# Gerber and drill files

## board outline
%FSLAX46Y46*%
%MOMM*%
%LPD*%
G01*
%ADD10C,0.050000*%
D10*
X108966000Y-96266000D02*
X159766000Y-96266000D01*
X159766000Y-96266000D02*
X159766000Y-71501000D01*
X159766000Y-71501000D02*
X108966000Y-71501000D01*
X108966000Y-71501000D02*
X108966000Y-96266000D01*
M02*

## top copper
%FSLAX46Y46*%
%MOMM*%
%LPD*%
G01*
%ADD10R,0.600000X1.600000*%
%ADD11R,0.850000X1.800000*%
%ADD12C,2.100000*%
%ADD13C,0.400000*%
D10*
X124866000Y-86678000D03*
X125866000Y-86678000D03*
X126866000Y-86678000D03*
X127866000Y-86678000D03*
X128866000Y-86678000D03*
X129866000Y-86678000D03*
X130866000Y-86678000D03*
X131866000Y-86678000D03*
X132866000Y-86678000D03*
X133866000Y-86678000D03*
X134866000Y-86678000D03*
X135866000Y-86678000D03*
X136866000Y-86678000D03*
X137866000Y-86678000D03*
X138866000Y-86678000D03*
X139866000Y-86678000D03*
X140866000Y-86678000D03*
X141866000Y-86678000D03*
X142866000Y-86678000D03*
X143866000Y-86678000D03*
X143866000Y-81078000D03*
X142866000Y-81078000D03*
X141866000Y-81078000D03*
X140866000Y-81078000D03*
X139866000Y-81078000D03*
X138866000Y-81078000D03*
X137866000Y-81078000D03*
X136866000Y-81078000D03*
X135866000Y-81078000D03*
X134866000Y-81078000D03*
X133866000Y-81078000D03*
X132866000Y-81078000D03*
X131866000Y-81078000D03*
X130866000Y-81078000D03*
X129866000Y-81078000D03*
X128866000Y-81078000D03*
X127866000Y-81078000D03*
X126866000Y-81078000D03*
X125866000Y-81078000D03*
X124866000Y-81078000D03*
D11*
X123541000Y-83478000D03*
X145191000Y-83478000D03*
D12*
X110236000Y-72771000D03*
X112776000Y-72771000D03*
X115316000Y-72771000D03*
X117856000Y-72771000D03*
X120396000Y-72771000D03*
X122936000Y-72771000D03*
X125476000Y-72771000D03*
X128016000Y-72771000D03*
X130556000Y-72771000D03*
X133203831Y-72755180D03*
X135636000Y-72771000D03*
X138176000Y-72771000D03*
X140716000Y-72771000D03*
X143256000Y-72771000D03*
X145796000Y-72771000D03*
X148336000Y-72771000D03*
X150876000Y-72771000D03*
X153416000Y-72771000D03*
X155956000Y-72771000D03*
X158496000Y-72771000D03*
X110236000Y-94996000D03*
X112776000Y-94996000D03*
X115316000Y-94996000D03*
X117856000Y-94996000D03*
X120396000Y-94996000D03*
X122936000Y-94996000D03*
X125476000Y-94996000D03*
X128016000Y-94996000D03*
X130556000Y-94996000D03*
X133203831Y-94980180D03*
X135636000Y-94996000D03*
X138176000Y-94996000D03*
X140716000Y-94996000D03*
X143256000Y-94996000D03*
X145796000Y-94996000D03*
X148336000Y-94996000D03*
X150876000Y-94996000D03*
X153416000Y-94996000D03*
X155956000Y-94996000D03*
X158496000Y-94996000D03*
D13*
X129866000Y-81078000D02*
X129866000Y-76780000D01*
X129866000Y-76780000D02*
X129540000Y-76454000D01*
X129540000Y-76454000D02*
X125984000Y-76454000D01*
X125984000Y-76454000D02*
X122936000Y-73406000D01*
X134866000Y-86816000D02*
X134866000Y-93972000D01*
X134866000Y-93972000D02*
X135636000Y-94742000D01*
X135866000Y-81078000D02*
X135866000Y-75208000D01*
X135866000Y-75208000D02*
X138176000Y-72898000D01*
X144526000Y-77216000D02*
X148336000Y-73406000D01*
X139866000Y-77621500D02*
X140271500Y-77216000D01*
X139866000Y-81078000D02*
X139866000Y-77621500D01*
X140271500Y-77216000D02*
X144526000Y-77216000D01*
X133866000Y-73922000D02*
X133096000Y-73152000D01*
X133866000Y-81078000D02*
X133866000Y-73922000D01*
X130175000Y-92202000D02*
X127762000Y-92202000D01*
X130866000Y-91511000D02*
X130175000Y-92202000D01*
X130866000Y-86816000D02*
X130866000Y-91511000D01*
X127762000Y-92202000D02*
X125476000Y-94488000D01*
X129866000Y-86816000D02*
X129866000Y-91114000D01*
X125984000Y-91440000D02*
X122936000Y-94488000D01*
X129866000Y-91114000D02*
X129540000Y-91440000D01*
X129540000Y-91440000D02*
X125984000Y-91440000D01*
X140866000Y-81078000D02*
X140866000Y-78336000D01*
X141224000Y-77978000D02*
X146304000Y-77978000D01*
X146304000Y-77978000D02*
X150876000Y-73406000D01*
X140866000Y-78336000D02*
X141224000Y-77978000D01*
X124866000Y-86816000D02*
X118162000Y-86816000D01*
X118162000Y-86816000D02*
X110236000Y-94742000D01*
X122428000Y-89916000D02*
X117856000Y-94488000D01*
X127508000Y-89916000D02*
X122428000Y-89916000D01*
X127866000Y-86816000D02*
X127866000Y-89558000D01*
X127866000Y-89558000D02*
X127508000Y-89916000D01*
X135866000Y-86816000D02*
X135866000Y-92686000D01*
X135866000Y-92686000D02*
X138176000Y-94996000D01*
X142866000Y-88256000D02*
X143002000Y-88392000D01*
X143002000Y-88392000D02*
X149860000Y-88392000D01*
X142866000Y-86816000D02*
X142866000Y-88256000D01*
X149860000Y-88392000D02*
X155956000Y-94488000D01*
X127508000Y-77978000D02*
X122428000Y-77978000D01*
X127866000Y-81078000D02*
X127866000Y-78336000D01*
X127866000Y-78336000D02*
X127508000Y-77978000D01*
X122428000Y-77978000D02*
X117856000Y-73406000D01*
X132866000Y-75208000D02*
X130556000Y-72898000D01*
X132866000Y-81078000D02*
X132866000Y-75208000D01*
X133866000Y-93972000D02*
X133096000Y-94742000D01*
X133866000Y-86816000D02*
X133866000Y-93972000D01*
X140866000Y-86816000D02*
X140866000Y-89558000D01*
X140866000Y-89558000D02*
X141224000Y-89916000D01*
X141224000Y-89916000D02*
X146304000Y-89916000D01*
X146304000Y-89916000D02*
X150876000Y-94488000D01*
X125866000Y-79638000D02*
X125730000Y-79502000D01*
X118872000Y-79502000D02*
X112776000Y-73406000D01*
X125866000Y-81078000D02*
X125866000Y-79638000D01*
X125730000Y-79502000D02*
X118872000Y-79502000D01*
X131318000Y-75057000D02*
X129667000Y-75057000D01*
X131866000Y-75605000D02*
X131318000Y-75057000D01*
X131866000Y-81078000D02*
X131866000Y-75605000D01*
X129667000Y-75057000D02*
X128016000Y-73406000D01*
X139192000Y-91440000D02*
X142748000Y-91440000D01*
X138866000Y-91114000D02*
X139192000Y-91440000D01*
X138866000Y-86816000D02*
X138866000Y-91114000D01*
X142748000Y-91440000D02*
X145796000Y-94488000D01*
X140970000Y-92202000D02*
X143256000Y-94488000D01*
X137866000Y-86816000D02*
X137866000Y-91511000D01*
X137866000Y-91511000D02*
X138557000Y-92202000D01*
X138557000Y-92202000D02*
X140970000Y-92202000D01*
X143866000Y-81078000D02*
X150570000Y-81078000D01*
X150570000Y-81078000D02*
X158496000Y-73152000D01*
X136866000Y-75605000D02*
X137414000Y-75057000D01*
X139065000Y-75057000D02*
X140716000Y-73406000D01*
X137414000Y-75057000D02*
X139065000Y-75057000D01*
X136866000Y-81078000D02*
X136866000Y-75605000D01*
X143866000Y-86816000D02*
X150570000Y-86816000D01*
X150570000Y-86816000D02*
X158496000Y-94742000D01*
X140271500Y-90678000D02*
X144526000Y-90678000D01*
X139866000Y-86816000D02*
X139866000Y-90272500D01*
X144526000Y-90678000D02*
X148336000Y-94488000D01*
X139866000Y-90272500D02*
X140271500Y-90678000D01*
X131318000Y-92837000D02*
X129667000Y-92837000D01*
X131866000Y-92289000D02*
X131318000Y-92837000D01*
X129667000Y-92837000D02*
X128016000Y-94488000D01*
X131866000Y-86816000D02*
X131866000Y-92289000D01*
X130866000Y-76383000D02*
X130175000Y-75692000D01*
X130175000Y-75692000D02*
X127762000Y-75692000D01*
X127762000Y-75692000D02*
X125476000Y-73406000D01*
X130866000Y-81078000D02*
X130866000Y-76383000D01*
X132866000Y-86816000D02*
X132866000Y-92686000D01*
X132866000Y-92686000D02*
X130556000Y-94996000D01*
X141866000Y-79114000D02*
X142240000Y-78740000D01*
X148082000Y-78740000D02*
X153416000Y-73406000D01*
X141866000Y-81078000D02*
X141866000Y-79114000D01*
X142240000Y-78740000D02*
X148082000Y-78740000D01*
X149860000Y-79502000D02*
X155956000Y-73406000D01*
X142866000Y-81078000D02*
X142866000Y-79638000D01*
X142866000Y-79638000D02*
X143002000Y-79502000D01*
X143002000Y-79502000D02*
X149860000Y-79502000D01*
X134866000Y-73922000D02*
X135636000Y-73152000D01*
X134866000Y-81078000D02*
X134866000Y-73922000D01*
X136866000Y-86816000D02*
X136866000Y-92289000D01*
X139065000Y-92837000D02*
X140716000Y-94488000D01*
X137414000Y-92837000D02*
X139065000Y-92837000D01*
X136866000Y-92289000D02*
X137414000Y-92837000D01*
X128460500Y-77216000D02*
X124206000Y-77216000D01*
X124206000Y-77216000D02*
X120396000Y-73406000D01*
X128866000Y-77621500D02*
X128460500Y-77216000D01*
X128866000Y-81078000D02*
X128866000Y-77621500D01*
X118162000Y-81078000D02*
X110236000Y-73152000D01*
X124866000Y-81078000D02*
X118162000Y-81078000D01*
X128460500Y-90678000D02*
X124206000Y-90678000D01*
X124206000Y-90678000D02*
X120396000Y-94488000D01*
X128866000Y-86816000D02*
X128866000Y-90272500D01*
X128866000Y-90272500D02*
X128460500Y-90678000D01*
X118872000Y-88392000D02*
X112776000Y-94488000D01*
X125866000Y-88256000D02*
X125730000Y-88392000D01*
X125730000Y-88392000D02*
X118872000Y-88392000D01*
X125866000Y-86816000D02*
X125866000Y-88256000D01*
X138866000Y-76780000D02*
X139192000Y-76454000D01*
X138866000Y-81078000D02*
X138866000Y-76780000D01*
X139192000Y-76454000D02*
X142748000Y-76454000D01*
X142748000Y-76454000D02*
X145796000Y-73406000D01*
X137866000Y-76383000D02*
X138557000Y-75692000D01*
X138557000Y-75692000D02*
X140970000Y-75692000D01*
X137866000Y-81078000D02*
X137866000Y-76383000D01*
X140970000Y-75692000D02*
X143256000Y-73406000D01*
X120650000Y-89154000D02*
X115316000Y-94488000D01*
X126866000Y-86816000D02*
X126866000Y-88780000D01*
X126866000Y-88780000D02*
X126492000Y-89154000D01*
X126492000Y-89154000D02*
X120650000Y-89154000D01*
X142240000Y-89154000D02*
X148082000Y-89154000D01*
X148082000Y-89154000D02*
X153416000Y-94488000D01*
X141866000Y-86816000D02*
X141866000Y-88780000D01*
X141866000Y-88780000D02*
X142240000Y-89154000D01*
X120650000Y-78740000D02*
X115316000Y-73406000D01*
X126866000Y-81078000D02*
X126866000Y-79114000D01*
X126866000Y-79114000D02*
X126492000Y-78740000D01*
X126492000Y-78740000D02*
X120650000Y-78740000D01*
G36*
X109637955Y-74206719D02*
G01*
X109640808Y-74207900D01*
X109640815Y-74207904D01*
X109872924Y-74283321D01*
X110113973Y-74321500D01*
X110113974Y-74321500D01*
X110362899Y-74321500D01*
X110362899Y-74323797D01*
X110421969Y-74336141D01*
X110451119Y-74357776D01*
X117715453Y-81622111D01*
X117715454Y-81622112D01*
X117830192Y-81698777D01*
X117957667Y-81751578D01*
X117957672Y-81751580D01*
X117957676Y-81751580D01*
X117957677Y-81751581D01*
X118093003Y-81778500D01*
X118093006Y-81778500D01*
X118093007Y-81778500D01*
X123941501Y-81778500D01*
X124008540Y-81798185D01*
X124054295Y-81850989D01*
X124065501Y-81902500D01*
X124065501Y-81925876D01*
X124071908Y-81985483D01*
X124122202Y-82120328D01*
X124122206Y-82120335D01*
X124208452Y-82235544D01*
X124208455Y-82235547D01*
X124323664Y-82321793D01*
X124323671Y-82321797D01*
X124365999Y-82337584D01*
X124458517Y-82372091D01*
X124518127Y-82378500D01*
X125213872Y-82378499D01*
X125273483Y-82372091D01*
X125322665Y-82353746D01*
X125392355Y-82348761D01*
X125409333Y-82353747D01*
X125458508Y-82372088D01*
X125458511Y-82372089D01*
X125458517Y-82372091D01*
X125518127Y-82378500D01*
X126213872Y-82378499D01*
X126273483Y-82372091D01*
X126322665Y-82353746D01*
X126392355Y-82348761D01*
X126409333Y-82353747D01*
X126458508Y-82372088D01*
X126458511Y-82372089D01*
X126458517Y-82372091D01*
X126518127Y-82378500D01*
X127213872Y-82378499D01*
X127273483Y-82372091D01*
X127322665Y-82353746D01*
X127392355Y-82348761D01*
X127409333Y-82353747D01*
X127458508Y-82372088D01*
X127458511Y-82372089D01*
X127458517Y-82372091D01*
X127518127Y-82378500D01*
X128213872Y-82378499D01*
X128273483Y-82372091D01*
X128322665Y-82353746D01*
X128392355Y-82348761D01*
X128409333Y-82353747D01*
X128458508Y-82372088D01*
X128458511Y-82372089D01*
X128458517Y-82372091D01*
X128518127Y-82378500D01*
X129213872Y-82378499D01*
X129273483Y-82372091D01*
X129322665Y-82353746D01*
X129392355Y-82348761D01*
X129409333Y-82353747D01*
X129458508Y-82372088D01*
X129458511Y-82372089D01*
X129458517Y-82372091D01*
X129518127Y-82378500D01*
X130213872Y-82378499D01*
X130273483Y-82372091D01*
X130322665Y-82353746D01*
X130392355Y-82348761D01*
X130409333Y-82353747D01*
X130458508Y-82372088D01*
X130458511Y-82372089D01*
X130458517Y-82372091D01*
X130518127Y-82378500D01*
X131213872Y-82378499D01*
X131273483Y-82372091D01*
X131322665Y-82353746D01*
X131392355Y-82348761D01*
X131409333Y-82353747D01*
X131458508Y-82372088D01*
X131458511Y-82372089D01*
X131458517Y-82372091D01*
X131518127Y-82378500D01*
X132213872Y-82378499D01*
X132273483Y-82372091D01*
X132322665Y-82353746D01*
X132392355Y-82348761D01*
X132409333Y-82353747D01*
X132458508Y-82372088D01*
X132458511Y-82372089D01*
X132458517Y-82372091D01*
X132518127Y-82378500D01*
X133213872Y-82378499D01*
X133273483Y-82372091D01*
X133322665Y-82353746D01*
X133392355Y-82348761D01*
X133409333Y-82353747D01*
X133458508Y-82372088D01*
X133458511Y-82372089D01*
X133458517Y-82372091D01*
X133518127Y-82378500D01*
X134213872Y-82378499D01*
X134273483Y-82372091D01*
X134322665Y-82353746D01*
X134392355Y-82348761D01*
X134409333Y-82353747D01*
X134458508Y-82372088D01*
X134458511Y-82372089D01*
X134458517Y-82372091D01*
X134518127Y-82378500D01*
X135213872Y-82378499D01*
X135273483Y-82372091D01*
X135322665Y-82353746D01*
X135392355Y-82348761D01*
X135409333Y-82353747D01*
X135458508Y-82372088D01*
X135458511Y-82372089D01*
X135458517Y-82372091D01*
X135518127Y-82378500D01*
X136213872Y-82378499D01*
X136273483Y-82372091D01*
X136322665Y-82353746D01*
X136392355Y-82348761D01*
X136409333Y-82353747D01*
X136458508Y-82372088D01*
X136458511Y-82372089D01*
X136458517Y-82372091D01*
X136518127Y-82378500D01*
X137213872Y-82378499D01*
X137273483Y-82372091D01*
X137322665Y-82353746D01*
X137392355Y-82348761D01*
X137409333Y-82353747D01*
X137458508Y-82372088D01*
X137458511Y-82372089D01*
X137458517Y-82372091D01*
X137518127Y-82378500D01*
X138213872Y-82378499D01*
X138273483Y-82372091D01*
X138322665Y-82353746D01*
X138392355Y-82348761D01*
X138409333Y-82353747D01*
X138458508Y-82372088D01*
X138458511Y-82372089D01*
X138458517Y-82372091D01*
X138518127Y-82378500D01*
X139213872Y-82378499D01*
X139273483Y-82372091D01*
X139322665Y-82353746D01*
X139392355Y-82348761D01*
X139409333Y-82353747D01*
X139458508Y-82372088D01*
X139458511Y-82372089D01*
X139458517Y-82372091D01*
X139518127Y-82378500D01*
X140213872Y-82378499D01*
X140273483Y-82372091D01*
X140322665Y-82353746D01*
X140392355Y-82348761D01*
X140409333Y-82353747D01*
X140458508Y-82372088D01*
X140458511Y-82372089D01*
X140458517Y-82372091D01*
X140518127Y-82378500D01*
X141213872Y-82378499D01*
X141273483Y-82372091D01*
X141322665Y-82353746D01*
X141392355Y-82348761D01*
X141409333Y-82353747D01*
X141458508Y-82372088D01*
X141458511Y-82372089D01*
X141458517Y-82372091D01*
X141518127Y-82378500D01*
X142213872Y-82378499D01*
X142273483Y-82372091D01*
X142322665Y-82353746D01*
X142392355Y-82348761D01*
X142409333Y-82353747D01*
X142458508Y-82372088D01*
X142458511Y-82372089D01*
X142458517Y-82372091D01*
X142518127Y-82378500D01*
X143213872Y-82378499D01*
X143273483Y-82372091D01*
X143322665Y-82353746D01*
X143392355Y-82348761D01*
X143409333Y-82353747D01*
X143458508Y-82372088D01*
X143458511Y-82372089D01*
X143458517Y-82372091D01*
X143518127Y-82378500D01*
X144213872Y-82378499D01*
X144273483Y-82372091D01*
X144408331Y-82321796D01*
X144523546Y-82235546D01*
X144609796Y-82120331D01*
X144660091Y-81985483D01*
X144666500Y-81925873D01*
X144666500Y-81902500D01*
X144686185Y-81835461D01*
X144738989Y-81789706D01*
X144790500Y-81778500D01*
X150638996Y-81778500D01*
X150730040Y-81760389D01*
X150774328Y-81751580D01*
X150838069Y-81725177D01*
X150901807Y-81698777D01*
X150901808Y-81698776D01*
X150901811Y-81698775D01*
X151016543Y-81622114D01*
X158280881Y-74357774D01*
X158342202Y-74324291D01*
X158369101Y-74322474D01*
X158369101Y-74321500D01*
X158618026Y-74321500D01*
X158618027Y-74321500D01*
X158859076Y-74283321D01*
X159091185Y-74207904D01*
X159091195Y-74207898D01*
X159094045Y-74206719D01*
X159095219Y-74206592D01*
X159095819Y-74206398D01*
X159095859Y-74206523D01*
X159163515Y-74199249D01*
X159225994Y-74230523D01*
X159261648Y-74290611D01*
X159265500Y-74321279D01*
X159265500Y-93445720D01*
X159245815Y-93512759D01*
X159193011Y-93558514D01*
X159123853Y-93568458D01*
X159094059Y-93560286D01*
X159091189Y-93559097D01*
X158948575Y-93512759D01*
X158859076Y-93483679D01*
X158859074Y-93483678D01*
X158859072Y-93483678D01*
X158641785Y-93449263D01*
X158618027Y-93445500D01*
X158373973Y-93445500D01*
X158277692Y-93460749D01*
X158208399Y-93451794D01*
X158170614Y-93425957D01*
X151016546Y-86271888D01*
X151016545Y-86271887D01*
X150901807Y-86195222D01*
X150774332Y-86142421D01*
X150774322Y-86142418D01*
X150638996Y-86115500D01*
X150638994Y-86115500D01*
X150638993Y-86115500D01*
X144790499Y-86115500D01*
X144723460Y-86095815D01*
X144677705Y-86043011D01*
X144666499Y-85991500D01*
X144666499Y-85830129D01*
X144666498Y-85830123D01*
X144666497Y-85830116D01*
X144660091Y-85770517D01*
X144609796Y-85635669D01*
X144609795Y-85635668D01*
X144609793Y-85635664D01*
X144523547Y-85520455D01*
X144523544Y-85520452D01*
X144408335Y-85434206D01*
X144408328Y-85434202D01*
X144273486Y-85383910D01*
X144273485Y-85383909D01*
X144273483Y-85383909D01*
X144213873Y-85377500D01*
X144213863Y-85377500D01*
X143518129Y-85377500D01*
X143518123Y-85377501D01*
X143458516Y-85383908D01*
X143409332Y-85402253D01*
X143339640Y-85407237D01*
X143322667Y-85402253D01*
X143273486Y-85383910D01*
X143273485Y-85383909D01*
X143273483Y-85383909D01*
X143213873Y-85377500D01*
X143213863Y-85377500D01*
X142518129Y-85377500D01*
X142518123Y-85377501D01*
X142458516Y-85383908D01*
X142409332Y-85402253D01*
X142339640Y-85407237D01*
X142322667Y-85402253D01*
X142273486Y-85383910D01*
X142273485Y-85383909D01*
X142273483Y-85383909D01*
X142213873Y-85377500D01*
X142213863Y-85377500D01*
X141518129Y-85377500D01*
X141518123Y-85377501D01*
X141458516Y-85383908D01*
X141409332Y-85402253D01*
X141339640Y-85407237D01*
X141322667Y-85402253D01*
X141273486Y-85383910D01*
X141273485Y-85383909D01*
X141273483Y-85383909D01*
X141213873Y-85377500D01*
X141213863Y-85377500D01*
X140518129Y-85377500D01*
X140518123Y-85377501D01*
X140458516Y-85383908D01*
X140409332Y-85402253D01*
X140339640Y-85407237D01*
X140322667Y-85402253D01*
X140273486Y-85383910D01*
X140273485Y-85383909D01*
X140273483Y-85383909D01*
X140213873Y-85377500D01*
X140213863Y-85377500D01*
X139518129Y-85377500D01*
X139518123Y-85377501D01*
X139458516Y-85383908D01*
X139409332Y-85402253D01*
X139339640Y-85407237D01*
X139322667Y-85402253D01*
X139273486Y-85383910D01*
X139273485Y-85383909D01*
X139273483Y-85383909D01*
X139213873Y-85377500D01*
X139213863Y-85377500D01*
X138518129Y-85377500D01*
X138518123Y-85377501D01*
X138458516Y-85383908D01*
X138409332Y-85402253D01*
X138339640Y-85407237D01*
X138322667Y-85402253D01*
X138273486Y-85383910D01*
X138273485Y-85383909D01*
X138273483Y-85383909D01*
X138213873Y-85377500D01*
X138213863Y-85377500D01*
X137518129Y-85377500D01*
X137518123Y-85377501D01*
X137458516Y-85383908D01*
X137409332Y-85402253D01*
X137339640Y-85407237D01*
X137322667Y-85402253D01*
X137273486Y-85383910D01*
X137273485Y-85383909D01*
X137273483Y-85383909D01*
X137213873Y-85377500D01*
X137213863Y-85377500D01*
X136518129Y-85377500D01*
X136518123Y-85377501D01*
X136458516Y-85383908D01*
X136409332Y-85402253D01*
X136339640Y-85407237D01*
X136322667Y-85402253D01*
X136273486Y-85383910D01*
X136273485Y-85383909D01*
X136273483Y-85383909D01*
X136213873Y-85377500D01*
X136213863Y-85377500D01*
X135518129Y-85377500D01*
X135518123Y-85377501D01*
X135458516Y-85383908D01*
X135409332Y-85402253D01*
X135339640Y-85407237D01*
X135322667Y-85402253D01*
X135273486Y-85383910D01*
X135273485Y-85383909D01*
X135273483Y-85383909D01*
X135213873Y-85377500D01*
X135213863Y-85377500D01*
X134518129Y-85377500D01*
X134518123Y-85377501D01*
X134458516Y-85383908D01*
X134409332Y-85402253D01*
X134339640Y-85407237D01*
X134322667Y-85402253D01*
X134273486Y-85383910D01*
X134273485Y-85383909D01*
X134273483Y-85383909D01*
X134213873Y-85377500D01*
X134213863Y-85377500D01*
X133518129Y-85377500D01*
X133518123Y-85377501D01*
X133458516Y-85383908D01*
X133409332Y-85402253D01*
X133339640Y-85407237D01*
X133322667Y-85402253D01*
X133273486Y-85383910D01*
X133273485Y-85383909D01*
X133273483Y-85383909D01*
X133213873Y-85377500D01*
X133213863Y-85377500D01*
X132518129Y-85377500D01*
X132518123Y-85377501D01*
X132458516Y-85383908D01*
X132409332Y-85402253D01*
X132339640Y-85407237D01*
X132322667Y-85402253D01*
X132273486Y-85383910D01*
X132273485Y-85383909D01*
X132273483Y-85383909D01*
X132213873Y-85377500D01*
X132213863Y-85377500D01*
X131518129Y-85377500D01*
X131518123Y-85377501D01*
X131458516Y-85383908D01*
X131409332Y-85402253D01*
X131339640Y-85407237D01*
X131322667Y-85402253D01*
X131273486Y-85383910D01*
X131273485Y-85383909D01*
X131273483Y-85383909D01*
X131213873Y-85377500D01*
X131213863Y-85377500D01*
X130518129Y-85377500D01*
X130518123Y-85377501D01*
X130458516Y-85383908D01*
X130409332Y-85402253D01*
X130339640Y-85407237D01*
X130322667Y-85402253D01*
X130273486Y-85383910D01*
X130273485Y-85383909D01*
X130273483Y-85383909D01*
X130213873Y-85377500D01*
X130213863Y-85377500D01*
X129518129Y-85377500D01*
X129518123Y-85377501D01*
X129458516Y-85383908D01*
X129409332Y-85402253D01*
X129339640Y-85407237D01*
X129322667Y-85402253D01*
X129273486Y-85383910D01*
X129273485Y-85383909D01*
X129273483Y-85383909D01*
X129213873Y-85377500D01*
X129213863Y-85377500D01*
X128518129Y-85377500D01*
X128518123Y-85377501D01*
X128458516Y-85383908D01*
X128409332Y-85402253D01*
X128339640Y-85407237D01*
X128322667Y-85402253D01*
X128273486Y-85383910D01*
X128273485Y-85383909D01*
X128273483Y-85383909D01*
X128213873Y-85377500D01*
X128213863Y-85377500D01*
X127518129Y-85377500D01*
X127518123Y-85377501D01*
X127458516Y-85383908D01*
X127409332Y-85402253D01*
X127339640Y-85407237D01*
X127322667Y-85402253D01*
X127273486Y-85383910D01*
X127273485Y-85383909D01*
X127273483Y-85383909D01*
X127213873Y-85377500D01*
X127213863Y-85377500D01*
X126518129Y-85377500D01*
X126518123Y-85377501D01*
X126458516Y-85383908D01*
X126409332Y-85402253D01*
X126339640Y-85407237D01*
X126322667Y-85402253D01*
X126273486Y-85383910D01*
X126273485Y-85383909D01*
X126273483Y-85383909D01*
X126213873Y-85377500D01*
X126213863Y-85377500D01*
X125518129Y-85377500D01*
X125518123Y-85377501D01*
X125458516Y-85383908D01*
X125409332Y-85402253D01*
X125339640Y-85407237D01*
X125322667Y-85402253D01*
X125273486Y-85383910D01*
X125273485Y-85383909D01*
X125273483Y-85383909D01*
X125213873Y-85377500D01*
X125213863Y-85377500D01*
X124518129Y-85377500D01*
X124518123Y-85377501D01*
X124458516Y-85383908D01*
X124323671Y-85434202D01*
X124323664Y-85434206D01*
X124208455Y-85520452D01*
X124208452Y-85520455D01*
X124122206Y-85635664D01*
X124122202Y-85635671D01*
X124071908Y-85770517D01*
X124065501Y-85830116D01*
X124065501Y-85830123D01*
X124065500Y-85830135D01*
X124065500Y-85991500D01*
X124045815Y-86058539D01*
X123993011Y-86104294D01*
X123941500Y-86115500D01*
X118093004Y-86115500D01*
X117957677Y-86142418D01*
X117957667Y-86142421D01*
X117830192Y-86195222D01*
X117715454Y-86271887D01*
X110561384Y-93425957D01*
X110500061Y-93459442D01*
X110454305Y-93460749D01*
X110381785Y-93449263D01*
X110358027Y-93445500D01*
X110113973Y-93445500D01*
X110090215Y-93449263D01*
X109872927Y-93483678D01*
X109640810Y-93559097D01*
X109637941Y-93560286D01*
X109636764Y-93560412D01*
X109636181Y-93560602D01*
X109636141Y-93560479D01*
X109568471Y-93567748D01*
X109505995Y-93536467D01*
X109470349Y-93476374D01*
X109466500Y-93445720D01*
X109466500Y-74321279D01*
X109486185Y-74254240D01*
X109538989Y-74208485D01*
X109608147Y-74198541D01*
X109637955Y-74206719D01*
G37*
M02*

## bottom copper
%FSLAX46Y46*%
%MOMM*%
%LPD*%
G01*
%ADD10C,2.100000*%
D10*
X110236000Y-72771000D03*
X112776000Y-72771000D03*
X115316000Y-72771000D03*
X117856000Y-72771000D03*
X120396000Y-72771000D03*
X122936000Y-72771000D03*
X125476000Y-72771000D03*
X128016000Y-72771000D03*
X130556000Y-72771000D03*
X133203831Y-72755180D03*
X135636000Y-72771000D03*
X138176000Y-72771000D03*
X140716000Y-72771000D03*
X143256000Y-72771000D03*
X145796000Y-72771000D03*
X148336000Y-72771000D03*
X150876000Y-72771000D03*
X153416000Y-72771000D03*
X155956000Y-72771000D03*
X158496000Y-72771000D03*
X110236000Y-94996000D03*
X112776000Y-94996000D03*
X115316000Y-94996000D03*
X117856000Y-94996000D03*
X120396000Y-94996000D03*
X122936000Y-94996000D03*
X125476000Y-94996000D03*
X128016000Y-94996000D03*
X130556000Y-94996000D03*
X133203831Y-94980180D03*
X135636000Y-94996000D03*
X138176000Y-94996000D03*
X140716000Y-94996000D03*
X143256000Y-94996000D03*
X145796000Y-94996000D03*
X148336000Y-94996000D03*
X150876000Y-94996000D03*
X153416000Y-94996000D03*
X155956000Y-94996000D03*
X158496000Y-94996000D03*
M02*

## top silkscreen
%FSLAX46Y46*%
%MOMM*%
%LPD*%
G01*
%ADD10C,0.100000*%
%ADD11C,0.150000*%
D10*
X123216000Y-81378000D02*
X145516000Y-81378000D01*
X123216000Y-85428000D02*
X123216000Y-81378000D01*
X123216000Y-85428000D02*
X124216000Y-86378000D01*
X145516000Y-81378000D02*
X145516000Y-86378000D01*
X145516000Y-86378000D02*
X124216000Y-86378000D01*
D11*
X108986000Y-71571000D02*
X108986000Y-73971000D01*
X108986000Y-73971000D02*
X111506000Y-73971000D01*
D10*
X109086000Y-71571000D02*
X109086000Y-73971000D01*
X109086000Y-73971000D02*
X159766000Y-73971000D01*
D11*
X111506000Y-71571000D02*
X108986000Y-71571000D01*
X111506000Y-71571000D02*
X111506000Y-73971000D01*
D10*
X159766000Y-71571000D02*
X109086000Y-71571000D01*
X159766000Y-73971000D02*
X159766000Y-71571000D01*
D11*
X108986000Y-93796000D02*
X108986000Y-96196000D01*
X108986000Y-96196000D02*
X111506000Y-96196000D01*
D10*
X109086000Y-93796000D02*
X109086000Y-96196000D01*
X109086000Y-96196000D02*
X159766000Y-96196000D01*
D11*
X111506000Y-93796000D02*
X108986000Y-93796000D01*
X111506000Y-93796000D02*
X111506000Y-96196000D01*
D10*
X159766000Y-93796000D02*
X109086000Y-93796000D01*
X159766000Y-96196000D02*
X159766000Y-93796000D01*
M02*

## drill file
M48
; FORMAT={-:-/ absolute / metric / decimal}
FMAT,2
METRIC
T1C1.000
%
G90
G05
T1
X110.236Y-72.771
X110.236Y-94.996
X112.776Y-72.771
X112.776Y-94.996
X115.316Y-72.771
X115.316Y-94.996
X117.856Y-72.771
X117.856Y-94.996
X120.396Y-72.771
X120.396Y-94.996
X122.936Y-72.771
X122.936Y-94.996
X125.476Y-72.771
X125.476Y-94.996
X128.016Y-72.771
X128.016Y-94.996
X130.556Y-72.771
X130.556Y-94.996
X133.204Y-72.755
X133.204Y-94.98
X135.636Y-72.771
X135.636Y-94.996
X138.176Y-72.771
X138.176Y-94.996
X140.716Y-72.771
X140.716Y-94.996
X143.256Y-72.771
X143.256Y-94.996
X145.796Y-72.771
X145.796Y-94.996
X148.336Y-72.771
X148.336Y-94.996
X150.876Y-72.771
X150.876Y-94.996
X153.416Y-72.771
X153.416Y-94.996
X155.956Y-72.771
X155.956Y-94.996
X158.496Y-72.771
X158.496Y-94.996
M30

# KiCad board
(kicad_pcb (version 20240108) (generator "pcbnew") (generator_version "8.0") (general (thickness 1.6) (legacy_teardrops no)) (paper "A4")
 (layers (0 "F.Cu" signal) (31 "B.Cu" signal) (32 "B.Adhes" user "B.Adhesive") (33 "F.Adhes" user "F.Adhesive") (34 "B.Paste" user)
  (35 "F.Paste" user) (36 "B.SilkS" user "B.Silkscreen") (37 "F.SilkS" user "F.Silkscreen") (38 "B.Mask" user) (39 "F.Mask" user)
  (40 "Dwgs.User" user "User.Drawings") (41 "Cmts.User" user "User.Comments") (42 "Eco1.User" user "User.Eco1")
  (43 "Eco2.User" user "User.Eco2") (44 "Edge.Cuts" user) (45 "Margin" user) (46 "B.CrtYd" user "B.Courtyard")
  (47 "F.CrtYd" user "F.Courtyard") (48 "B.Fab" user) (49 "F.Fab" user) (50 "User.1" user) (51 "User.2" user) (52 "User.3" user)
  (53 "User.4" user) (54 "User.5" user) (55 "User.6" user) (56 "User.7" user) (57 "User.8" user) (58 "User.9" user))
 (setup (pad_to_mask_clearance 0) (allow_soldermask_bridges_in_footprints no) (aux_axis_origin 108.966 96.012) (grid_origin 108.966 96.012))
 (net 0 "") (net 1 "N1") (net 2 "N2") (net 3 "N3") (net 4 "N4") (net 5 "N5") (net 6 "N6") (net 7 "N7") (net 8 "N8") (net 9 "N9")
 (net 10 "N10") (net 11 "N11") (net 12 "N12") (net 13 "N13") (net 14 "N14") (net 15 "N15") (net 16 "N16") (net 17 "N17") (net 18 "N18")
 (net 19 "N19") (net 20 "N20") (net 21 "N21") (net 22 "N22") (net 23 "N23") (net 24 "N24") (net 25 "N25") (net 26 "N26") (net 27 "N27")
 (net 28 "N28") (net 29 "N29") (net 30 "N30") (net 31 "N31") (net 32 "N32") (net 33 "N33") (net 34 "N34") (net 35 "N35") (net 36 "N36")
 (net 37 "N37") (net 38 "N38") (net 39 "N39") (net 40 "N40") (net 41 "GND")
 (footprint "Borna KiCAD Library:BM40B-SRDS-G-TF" (layer "F.Cu") (at 134.366 83.878)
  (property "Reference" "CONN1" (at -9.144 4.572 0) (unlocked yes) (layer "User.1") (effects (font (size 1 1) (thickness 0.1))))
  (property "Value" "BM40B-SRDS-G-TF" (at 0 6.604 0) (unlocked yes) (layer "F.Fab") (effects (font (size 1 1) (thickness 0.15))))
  (fp_line (start -11.15 -2.5) (end 11.15 -2.5) (stroke (width 0.1) (type default)) (layer "F.SilkS"))
  (fp_line (start -11.15 1.55) (end -11.15 -2.5) (stroke (width 0.1) (type default)) (layer "F.SilkS"))
  (fp_line (start -11.15 1.55) (end -10.15 2.5) (stroke (width 0.1) (type default)) (layer "F.SilkS"))
  (fp_line (start 11.15 -2.5) (end 11.15 2.5) (stroke (width 0.1) (type default)) (layer "F.SilkS"))
  (fp_line (start 11.15 2.5) (end -10.15 2.5) (stroke (width 0.1) (type default)) (layer "F.SilkS"))
  (pad "1" smd rect (at -9.5 2.8) (size 0.6 1.6) (layers "F.Cu" "F.Paste" "F.Mask") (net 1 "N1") (thermal_bridge_angle 45))
  (pad "2" smd rect (at -8.5 2.8) (size 0.6 1.6) (layers "F.Cu" "F.Paste" "F.Mask") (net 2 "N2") (thermal_bridge_angle 45))
  (pad "3" smd rect (at -7.5 2.8) (size 0.6 1.6) (layers "F.Cu" "F.Paste" "F.Mask") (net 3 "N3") (thermal_bridge_angle 45))
  (pad "4" smd rect (at -6.5 2.8) (size 0.6 1.6) (layers "F.Cu" "F.Paste" "F.Mask") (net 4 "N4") (thermal_bridge_angle 45))
  (pad "5" smd rect (at -5.5 2.8) (size 0.6 1.6) (layers "F.Cu" "F.Paste" "F.Mask") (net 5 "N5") (thermal_bridge_angle 45))
  (pad "6" smd rect (at -4.5 2.8) (size 0.6 1.6) (layers "F.Cu" "F.Paste" "F.Mask") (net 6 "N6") (thermal_bridge_angle 45))
  (pad "7" smd rect (at -3.5 2.8) (size 0.6 1.6) (layers "F.Cu" "F.Paste" "F.Mask") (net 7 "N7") (thermal_bridge_angle 45))
  (pad "8" smd rect (at -2.5 2.8) (size 0.6 1.6) (layers "F.Cu" "F.Paste" "F.Mask") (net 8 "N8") (thermal_bridge_angle 45))
  (pad "9" smd rect (at -1.5 2.8) (size 0.6 1.6) (layers "F.Cu" "F.Paste" "F.Mask") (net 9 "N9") (thermal_bridge_angle 45))
  (pad "10" smd rect (at -0.5 2.8) (size 0.6 1.6) (layers "F.Cu" "F.Paste" "F.Mask") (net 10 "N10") (thermal_bridge_angle 45))
  (pad "11" smd rect (at 0.5 2.8) (size 0.6 1.6) (layers "F.Cu" "F.Paste" "F.Mask") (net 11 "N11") (thermal_bridge_angle 45))
  (pad "12" smd rect (at 1.5 2.8) (size 0.6 1.6) (layers "F.Cu" "F.Paste" "F.Mask") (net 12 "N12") (thermal_bridge_angle 45))
  (pad "13" smd rect (at 2.5 2.8) (size 0.6 1.6) (layers "F.Cu" "F.Paste" "F.Mask") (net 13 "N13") (thermal_bridge_angle 45))
  (pad "14" smd rect (at 3.5 2.8) (size 0.6 1.6) (layers "F.Cu" "F.Paste" "F.Mask") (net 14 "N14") (thermal_bridge_angle 45))
  (pad "15" smd rect (at 4.5 2.8) (size 0.6 1.6) (layers "F.Cu" "F.Paste" "F.Mask") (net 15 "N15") (thermal_bridge_angle 45))
  (pad "16" smd rect (at 5.5 2.8) (size 0.6 1.6) (layers "F.Cu" "F.Paste" "F.Mask") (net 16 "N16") (thermal_bridge_angle 45))
  (pad "17" smd rect (at 6.5 2.8) (size 0.6 1.6) (layers "F.Cu" "F.Paste" "F.Mask") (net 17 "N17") (thermal_bridge_angle 45))
  (pad "18" smd rect (at 7.5 2.8) (size 0.6 1.6) (layers "F.Cu" "F.Paste" "F.Mask") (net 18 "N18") (thermal_bridge_angle 45))
  (pad "19" smd rect (at 8.5 2.8) (size 0.6 1.6) (layers "F.Cu" "F.Paste" "F.Mask") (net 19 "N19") (thermal_bridge_angle 45))
  (pad "20" smd rect (at 9.5 2.8) (size 0.6 1.6) (layers "F.Cu" "F.Paste" "F.Mask") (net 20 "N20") (thermal_bridge_angle 45))
  (pad "21" smd rect (at 9.5 -2.8) (size 0.6 1.6) (layers "F.Cu" "F.Paste" "F.Mask") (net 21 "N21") (thermal_bridge_angle 45))
  (pad "22" smd rect (at 8.5 -2.8) (size 0.6 1.6) (layers "F.Cu" "F.Paste" "F.Mask") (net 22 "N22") (thermal_bridge_angle 45))
  (pad "23" smd rect (at 7.5 -2.8) (size 0.6 1.6) (layers "F.Cu" "F.Paste" "F.Mask") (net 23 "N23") (thermal_bridge_angle 45))
  (pad "24" smd rect (at 6.5 -2.8) (size 0.6 1.6) (layers "F.Cu" "F.Paste" "F.Mask") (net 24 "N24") (thermal_bridge_angle 45))
  (pad "25" smd rect (at 5.5 -2.8) (size 0.6 1.6) (layers "F.Cu" "F.Paste" "F.Mask") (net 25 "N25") (thermal_bridge_angle 45))
  (pad "26" smd rect (at 4.5 -2.8) (size 0.6 1.6) (layers "F.Cu" "F.Paste" "F.Mask") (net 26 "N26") (thermal_bridge_angle 45))
  (pad "27" smd rect (at 3.5 -2.8) (size 0.6 1.6) (layers "F.Cu" "F.Paste" "F.Mask") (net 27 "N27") (thermal_bridge_angle 45))
  (pad "28" smd rect (at 2.5 -2.8) (size 0.6 1.6) (layers "F.Cu" "F.Paste" "F.Mask") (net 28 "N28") (thermal_bridge_angle 45))
  (pad "29" smd rect (at 1.5 -2.8) (size 0.6 1.6) (layers "F.Cu" "F.Paste" "F.Mask") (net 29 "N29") (thermal_bridge_angle 45))
  (pad "30" smd rect (at 0.5 -2.8) (size 0.6 1.6) (layers "F.Cu" "F.Paste" "F.Mask") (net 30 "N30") (thermal_bridge_angle 45))
  (pad "31" smd rect (at -0.5 -2.8) (size 0.6 1.6) (layers "F.Cu" "F.Paste" "F.Mask") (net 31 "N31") (thermal_bridge_angle 45))
  (pad "32" smd rect (at -1.5 -2.8) (size 0.6 1.6) (layers "F.Cu" "F.Paste" "F.Mask") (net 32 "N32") (thermal_bridge_angle 45))
  (pad "33" smd rect (at -2.5 -2.8) (size 0.6 1.6) (layers "F.Cu" "F.Paste" "F.Mask") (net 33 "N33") (thermal_bridge_angle 45))
  (pad "34" smd rect (at -3.5 -2.8) (size 0.6 1.6) (layers "F.Cu" "F.Paste" "F.Mask") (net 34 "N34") (thermal_bridge_angle 45))
  (pad "35" smd rect (at -4.5 -2.8) (size 0.6 1.6) (layers "F.Cu" "F.Paste" "F.Mask") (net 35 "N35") (thermal_bridge_angle 45))
  (pad "36" smd rect (at -5.5 -2.8) (size 0.6 1.6) (layers "F.Cu" "F.Paste" "F.Mask") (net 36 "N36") (thermal_bridge_angle 45))
  (pad "37" smd rect (at -6.5 -2.8) (size 0.6 1.6) (layers "F.Cu" "F.Paste" "F.Mask") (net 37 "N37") (thermal_bridge_angle 45))
  (pad "38" smd rect (at -7.5 -2.8) (size 0.6 1.6) (layers "F.Cu" "F.Paste" "F.Mask") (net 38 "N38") (thermal_bridge_angle 45))
  (pad "39" smd rect (at -8.5 -2.8) (size 0.6 1.6) (layers "F.Cu" "F.Paste" "F.Mask") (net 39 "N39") (thermal_bridge_angle 45))
  (pad "40" smd rect (at -9.5 -2.8) (size 0.6 1.6) (layers "F.Cu" "F.Paste" "F.Mask") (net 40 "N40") (thermal_bridge_angle 45))
  (pad "41" smd rect (at -10.825 -0.4) (size 0.85 1.8) (layers "F.Cu" "F.Paste" "F.Mask") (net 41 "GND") (thermal_bridge_angle 45))
  (pad "42" smd rect (at 10.825 -0.4) (size 0.85 1.8) (layers "F.Cu" "F.Paste" "F.Mask") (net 41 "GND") (thermal_bridge_angle 45)))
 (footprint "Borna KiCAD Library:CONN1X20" (layer "F.Cu") (at 134.366 72.771)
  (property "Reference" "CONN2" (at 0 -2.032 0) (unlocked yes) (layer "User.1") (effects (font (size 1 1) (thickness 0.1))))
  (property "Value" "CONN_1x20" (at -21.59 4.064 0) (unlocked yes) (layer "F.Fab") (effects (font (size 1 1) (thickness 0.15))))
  (fp_line (start -25.38 -1.2) (end -25.38 1.2) (stroke (width 0.15) (type default)) (layer "F.SilkS"))
  (fp_line (start -25.38 1.2) (end -22.86 1.2) (stroke (width 0.15) (type default)) (layer "F.SilkS"))
  (fp_line (start -25.28 -1.2) (end -25.28 1.2) (stroke (width 0.1) (type default)) (layer "F.SilkS"))
  (fp_line (start -25.28 1.2) (end 25.4 1.2) (stroke (width 0.1) (type default)) (layer "F.SilkS"))
  (fp_line (start -22.86 -1.2) (end -25.38 -1.2) (stroke (width 0.15) (type default)) (layer "F.SilkS"))
  (fp_line (start -22.86 -1.2) (end -22.86 1.2) (stroke (width 0.15) (type default)) (layer "F.SilkS"))
  (fp_line (start 25.4 -1.2) (end -25.28 -1.2) (stroke (width 0.1) (type default)) (layer "F.SilkS"))
  (fp_line (start 25.4 1.2) (end 25.4 -1.2) (stroke (width 0.1) (type default)) (layer "F.SilkS"))
  (pad "1" thru_hole circle (at -24.13 0) (size 2.1 2.1) (drill 1) (layers "*.Cu" "*.Mask") (remove_unused_layers no) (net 40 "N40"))
  (pad "2" thru_hole circle (at -21.59 0) (size 2.1 2.1) (drill 1) (layers "*.Cu" "*.Mask") (remove_unused_layers no) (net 39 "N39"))
  (pad "3" thru_hole circle (at -19.05 0) (size 2.1 2.1) (drill 1) (layers "*.Cu" "*.Mask") (remove_unused_layers no) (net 38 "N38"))
  (pad "4" thru_hole circle (at -16.51 0) (size 2.1 2.1) (drill 1) (layers "*.Cu" "*.Mask") (remove_unused_layers no) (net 37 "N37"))
  (pad "5" thru_hole circle (at -13.97 0) (size 2.1 2.1) (drill 1) (layers "*.Cu" "*.Mask") (remove_unused_layers no) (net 36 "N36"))
  (pad "6" thru_hole circle (at -11.43 0) (size 2.1 2.1) (drill 1) (layers "*.Cu" "*.Mask") (remove_unused_layers no) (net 35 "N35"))
  (pad "7" thru_hole circle (at -8.89 0) (size 2.1 2.1) (drill 1) (layers "*.Cu" "*.Mask") (remove_unused_layers no) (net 34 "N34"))
  (pad "8" thru_hole circle (at -6.35 0) (size 2.1 2.1) (drill 1) (layers "*.Cu" "*.Mask") (remove_unused_layers no) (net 33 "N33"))
  (pad "9" thru_hole circle (at -3.81 0) (size 2.1 2.1) (drill 1) (layers "*.Cu" "*.Mask") (remove_unused_layers no) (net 32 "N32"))
  (pad "10" thru_hole circle (at -1.162169 -0.01582) (size 2.1 2.1) (drill 1) (layers "*.Cu" "*.Mask") (remove_unused_layers no)
   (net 31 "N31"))
  (pad "11" thru_hole circle (at 1.27 0) (size 2.1 2.1) (drill 1) (layers "*.Cu" "*.Mask") (remove_unused_layers no) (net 30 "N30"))
  (pad "12" thru_hole circle (at 3.81 0) (size 2.1 2.1) (drill 1) (layers "*.Cu" "*.Mask") (remove_unused_layers no) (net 29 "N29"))
  (pad "13" thru_hole circle (at 6.35 0) (size 2.1 2.1) (drill 1) (layers "*.Cu" "*.Mask") (remove_unused_layers no) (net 28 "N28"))
  (pad "14" thru_hole circle (at 8.89 0) (size 2.1 2.1) (drill 1) (layers "*.Cu" "*.Mask") (remove_unused_layers no) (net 27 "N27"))
  (pad "15" thru_hole circle (at 11.43 0) (size 2.1 2.1) (drill 1) (layers "*.Cu" "*.Mask") (remove_unused_layers no) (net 26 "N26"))
  (pad "16" thru_hole circle (at 13.97 0) (size 2.1 2.1) (drill 1) (layers "*.Cu" "*.Mask") (remove_unused_layers no) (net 25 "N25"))
  (pad "17" thru_hole circle (at 16.51 0) (size 2.1 2.1) (drill 1) (layers "*.Cu" "*.Mask") (remove_unused_layers no) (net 24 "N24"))
  (pad "18" thru_hole circle (at 19.05 0) (size 2.1 2.1) (drill 1) (layers "*.Cu" "*.Mask") (remove_unused_layers no) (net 23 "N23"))
  (pad "19" thru_hole circle (at 21.59 0) (size 2.1 2.1) (drill 1) (layers "*.Cu" "*.Mask") (remove_unused_layers no) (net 22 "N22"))
  (pad "20" thru_hole circle (at 24.13 0) (size 2.1 2.1) (drill 1) (layers "*.Cu" "*.Mask") (remove_unused_layers no) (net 21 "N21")))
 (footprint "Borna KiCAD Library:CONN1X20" (layer "F.Cu") (at 134.366 94.996)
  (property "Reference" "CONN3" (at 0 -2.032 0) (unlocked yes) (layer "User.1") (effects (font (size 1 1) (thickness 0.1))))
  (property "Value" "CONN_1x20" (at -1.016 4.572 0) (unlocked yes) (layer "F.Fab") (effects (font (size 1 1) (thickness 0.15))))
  (fp_line (start -25.38 -1.2) (end -25.38 1.2) (stroke (width 0.15) (type default)) (layer "F.SilkS"))
  (fp_line (start -25.38 1.2) (end -22.86 1.2) (stroke (width 0.15) (type default)) (layer "F.SilkS"))
  (fp_line (start -25.28 -1.2) (end -25.28 1.2) (stroke (width 0.1) (type default)) (layer "F.SilkS"))
  (fp_line (start -25.28 1.2) (end 25.4 1.2) (stroke (width 0.1) (type default)) (layer "F.SilkS"))
  (fp_line (start -22.86 -1.2) (end -25.38 -1.2) (stroke (width 0.15) (type default)) (layer "F.SilkS"))
  (fp_line (start -22.86 -1.2) (end -22.86 1.2) (stroke (width 0.15) (type default)) (layer "F.SilkS"))
  (fp_line (start 25.4 -1.2) (end -25.28 -1.2) (stroke (width 0.1) (type default)) (layer "F.SilkS"))
  (fp_line (start 25.4 1.2) (end 25.4 -1.2) (stroke (width 0.1) (type default)) (layer "F.SilkS"))
  (pad "1" thru_hole circle (at -24.13 0) (size 2.1 2.1) (drill 1) (layers "*.Cu" "*.Mask") (remove_unused_layers no) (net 1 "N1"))
  (pad "2" thru_hole circle (at -21.59 0) (size 2.1 2.1) (drill 1) (layers "*.Cu" "*.Mask") (remove_unused_layers no) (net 2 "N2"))
  (pad "3" thru_hole circle (at -19.05 0) (size 2.1 2.1) (drill 1) (layers "*.Cu" "*.Mask") (remove_unused_layers no) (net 3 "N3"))
  (pad "4" thru_hole circle (at -16.51 0) (size 2.1 2.1) (drill 1) (layers "*.Cu" "*.Mask") (remove_unused_layers no) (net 4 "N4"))
  (pad "5" thru_hole circle (at -13.97 0) (size 2.1 2.1) (drill 1) (layers "*.Cu" "*.Mask") (remove_unused_layers no) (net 5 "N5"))
  (pad "6" thru_hole circle (at -11.43 0) (size 2.1 2.1) (drill 1) (layers "*.Cu" "*.Mask") (remove_unused_layers no) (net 6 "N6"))
  (pad "7" thru_hole circle (at -8.89 0) (size 2.1 2.1) (drill 1) (layers "*.Cu" "*.Mask") (remove_unused_layers no) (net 7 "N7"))
  (pad "8" thru_hole circle (at -6.35 0) (size 2.1 2.1) (drill 1) (layers "*.Cu" "*.Mask") (remove_unused_layers no) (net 8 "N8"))
  (pad "9" thru_hole circle (at -3.81 0) (size 2.1 2.1) (drill 1) (layers "*.Cu" "*.Mask") (remove_unused_layers no) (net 9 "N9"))
  (pad "10" thru_hole circle (at -1.162169 -0.01582) (size 2.1 2.1) (drill 1) (layers "*.Cu" "*.Mask") (remove_unused_layers no)
   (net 10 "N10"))
  (pad "11" thru_hole circle (at 1.27 0) (size 2.1 2.1) (drill 1) (layers "*.Cu" "*.Mask") (remove_unused_layers no) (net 11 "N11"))
  (pad "12" thru_hole circle (at 3.81 0) (size 2.1 2.1) (drill 1) (layers "*.Cu" "*.Mask") (remove_unused_layers no) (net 12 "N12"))
  (pad "13" thru_hole circle (at 6.35 0) (size 2.1 2.1) (drill 1) (layers "*.Cu" "*.Mask") (remove_unused_layers no) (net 13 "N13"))
  (pad "14" thru_hole circle (at 8.89 0) (size 2.1 2.1) (drill 1) (layers "*.Cu" "*.Mask") (remove_unused_layers no) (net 14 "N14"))
  (pad "15" thru_hole circle (at 11.43 0) (size 2.1 2.1) (drill 1) (layers "*.Cu" "*.Mask") (remove_unused_layers no) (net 15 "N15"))
  (pad "16" thru_hole circle (at 13.97 0) (size 2.1 2.1) (drill 1) (layers "*.Cu" "*.Mask") (remove_unused_layers no) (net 16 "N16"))
  (pad "17" thru_hole circle (at 16.51 0) (size 2.1 2.1) (drill 1) (layers "*.Cu" "*.Mask") (remove_unused_layers no) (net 17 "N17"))
  (pad "18" thru_hole circle (at 19.05 0) (size 2.1 2.1) (drill 1) (layers "*.Cu" "*.Mask") (remove_unused_layers no) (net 18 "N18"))
  (pad "19" thru_hole circle (at 21.59 0) (size 2.1 2.1) (drill 1) (layers "*.Cu" "*.Mask") (remove_unused_layers no) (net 19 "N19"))
  (pad "20" thru_hole circle (at 24.13 0) (size 2.1 2.1) (drill 1) (layers "*.Cu" "*.Mask") (remove_unused_layers no) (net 20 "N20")))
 (gr_line (start 108.966 96.266) (end 159.766 96.266) (stroke (width 0.05) (type default)) (layer "Edge.Cuts"))
 (gr_line (start 159.766 96.266) (end 159.766 71.501) (stroke (width 0.05) (type default)) (layer "Edge.Cuts"))
 (gr_line (start 159.766 71.501) (end 108.966 71.501) (stroke (width 0.05) (type default)) (layer "Edge.Cuts"))
 (gr_line (start 108.966 71.501) (end 108.966 96.266) (stroke (width 0.05) (type default)) (layer "Edge.Cuts"))
 (segment (start 129.866 81.078) (end 129.866 76.78) (width 0.4) (layer "F.Cu") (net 35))
 (segment (start 129.866 76.78) (end 129.54 76.454) (width 0.4) (layer "F.Cu") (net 35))
 (segment (start 129.54 76.454) (end 125.984 76.454) (width 0.4) (layer "F.Cu") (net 35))
 (segment (start 125.984 76.454) (end 122.936 73.406) (width 0.4) (layer "F.Cu") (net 35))
 (segment (start 134.866 86.816) (end 134.866 93.972) (width 0.4) (layer "F.Cu") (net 11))
 (segment (start 134.866 93.972) (end 135.636 94.742) (width 0.4) (layer "F.Cu") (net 11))
 (segment (start 135.866 81.078) (end 135.866 75.208) (width 0.4) (layer "F.Cu") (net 29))
 (segment (start 135.866 75.208) (end 138.176 72.898) (width 0.4) (layer "F.Cu") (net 29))
 (segment (start 144.526 77.216) (end 148.336 73.406) (width 0.4) (layer "F.Cu") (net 25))
 (segment (start 139.866 77.6215) (end 140.2715 77.216) (width 0.4) (layer "F.Cu") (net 25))
 (segment (start 139.866 81.078) (end 139.866 77.6215) (width 0.4) (layer "F.Cu") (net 25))
 (segment (start 140.2715 77.216) (end 144.526 77.216) (width 0.4) (layer "F.Cu") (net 25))
 (segment (start 133.866 73.922) (end 133.096 73.152) (width 0.4) (layer "F.Cu") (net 31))
 (segment (start 133.866 81.078) (end 133.866 73.922) (width 0.4) (layer "F.Cu") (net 31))
 (segment (start 130.175 92.202) (end 127.762 92.202) (width 0.4) (layer "F.Cu") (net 7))
 (segment (start 130.866 91.511) (end 130.175 92.202) (width 0.4) (layer "F.Cu") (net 7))
 (segment (start 130.866 86.816) (end 130.866 91.511) (width 0.4) (layer "F.Cu") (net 7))
 (segment (start 127.762 92.202) (end 125.476 94.488) (width 0.4) (layer "F.Cu") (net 7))
 (segment (start 129.866 86.816) (end 129.866 91.114) (width 0.4) (layer "F.Cu") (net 6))
 (segment (start 125.984 91.44) (end 122.936 94.488) (width 0.4) (layer "F.Cu") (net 6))
 (segment (start 129.866 91.114) (end 129.54 91.44) (width 0.4) (layer "F.Cu") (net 6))
 (segment (start 129.54 91.44) (end 125.984 91.44) (width 0.4) (layer "F.Cu") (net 6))
 (segment (start 140.866 81.078) (end 140.866 78.336) (width 0.4) (layer "F.Cu") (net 24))
 (segment (start 141.224 77.978) (end 146.304 77.978) (width 0.4) (layer "F.Cu") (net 24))
 (segment (start 146.304 77.978) (end 150.876 73.406) (width 0.4) (layer "F.Cu") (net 24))
 (segment (start 140.866 78.336) (end 141.224 77.978) (width 0.4) (layer "F.Cu") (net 24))
 (segment (start 124.866 86.816) (end 118.162 86.816) (width 0.4) (layer "F.Cu") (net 1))
 (segment (start 118.162 86.816) (end 110.236 94.742) (width 0.4) (layer "F.Cu") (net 1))
 (segment (start 122.428 89.916) (end 117.856 94.488) (width 0.4) (layer "F.Cu") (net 4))
 (segment (start 127.508 89.916) (end 122.428 89.916) (width 0.4) (layer "F.Cu") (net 4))
 (segment (start 127.866 86.816) (end 127.866 89.558) (width 0.4) (layer "F.Cu") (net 4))
 (segment (start 127.866 89.558) (end 127.508 89.916) (width 0.4) (layer "F.Cu") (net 4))
 (segment (start 135.866 86.816) (end 135.866 92.686) (width 0.4) (layer "F.Cu") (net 12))
 (segment (start 135.866 92.686) (end 138.176 94.996) (width 0.4) (layer "F.Cu") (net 12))
 (segment (start 142.866 88.256) (end 143.002 88.392) (width 0.4) (layer "F.Cu") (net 19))
 (segment (start 143.002 88.392) (end 149.86 88.392) (width 0.4) (layer "F.Cu") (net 19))
 (segment (start 142.866 86.816) (end 142.866 88.256) (width 0.4) (layer "F.Cu") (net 19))
 (segment (start 149.86 88.392) (end 155.956 94.488) (width 0.4) (layer "F.Cu") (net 19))
 (segment (start 127.508 77.978) (end 122.428 77.978) (width 0.4) (layer "F.Cu") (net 37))
 (segment (start 127.866 81.078) (end 127.866 78.336) (width 0.4) (layer "F.Cu") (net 37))
 (segment (start 127.866 78.336) (end 127.508 77.978) (width 0.4) (layer "F.Cu") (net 37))
 (segment (start 122.428 77.978) (end 117.856 73.406) (width 0.4) (layer "F.Cu") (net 37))
 (segment (start 132.866 75.208) (end 130.556 72.898) (width 0.4) (layer "F.Cu") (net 32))
 (segment (start 132.866 81.078) (end 132.866 75.208) (width 0.4) (layer "F.Cu") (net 32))
 (segment (start 133.866 93.972) (end 133.096 94.742) (width 0.4) (layer "F.Cu") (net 10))
 (segment (start 133.866 86.816) (end 133.866 93.972) (width 0.4) (layer "F.Cu") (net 10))
 (segment (start 140.866 86.816) (end 140.866 89.558) (width 0.4) (layer "F.Cu") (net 17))
 (segment (start 140.866 89.558) (end 141.224 89.916) (width 0.4) (layer "F.Cu") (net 17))
 (segment (start 141.224 89.916) (end 146.304 89.916) (width 0.4) (layer "F.Cu") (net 17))
 (segment (start 146.304 89.916) (end 150.876 94.488) (width 0.4) (layer "F.Cu") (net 17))
 (segment (start 125.866 79.638) (end 125.73 79.502) (width 0.4) (layer "F.Cu") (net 39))
 (segment (start 118.872 79.502) (end 112.776 73.406) (width 0.4) (layer "F.Cu") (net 39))
 (segment (start 125.866 81.078) (end 125.866 79.638) (width 0.4) (layer "F.Cu") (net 39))
 (segment (start 125.73 79.502) (end 118.872 79.502) (width 0.4) (layer "F.Cu") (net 39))
 (segment (start 131.318 75.057) (end 129.667 75.057) (width 0.4) (layer "F.Cu") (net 33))
 (segment (start 131.866 75.605) (end 131.318 75.057) (width 0.4) (layer "F.Cu") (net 33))
 (segment (start 131.866 81.078) (end 131.866 75.605) (width 0.4) (layer "F.Cu") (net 33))
 (segment (start 129.667 75.057) (end 128.016 73.406) (width 0.4) (layer "F.Cu") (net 33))
 (segment (start 139.192 91.44) (end 142.748 91.44) (width 0.4) (layer "F.Cu") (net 15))
 (segment (start 138.866 91.114) (end 139.192 91.44) (width 0.4) (layer "F.Cu") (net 15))
 (segment (start 138.866 86.816) (end 138.866 91.114) (width 0.4) (layer "F.Cu") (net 15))
 (segment (start 142.748 91.44) (end 145.796 94.488) (width 0.4) (layer "F.Cu") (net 15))
 (segment (start 140.97 92.202) (end 143.256 94.488) (width 0.4) (layer "F.Cu") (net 14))
 (segment (start 137.866 86.816) (end 137.866 91.511) (width 0.4) (layer "F.Cu") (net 14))
 (segment (start 137.866 91.511) (end 138.557 92.202) (width 0.4) (layer "F.Cu") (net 14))
 (segment (start 138.557 92.202) (end 140.97 92.202) (width 0.4) (layer "F.Cu") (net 14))
 (segment (start 143.866 81.078) (end 150.57 81.078) (width 0.4) (layer "F.Cu") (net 21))
 (segment (start 150.57 81.078) (end 158.496 73.152) (width 0.4) (layer "F.Cu") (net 21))
 (segment (start 136.866 75.605) (end 137.414 75.057) (width 0.4) (layer "F.Cu") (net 28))
 (segment (start 139.065 75.057) (end 140.716 73.406) (width 0.4) (layer "F.Cu") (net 28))
 (segment (start 137.414 75.057) (end 139.065 75.057) (width 0.4) (layer "F.Cu") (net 28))
 (segment (start 136.866 81.078) (end 136.866 75.605) (width 0.4) (layer "F.Cu") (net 28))
 (segment (start 143.866 86.816) (end 150.57 86.816) (width 0.4) (layer "F.Cu") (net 20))
 (segment (start 150.57 86.816) (end 158.496 94.742) (width 0.4) (layer "F.Cu") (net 20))
 (segment (start 140.2715 90.678) (end 144.526 90.678) (width 0.4) (layer "F.Cu") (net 16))
 (segment (start 139.866 86.816) (end 139.866 90.2725) (width 0.4) (layer "F.Cu") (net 16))
 (segment (start 144.526 90.678) (end 148.336 94.488) (width 0.4) (layer "F.Cu") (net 16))
 (segment (start 139.866 90.2725) (end 140.2715 90.678) (width 0.4) (layer "F.Cu") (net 16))
 (segment (start 131.318 92.837) (end 129.667 92.837) (width 0.4) (layer "F.Cu") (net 8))
 (segment (start 131.866 92.289) (end 131.318 92.837) (width 0.4) (layer "F.Cu") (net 8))
 (segment (start 129.667 92.837) (end 128.016 94.488) (width 0.4) (layer "F.Cu") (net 8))
 (segment (start 131.866 86.816) (end 131.866 92.289) (width 0.4) (layer "F.Cu") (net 8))
 (segment (start 130.866 76.383) (end 130.175 75.692) (width 0.4) (layer "F.Cu") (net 34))
 (segment (start 130.175 75.692) (end 127.762 75.692) (width 0.4) (layer "F.Cu") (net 34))
 (segment (start 127.762 75.692) (end 125.476 73.406) (width 0.4) (layer "F.Cu") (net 34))
 (segment (start 130.866 81.078) (end 130.866 76.383) (width 0.4) (layer "F.Cu") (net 34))
 (segment (start 132.866 86.816) (end 132.866 92.686) (width 0.4) (layer "F.Cu") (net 9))
 (segment (start 132.866 92.686) (end 130.556 94.996) (width 0.4) (layer "F.Cu") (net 9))
 (segment (start 141.866 79.114) (end 142.24 78.74) (width 0.4) (layer "F.Cu") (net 23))
 (segment (start 148.082 78.74) (end 153.416 73.406) (width 0.4) (layer "F.Cu") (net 23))
 (segment (start 141.866 81.078) (end 141.866 79.114) (width 0.4) (layer "F.Cu") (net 23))
 (segment (start 142.24 78.74) (end 148.082 78.74) (width 0.4) (layer "F.Cu") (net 23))
 (segment (start 149.86 79.502) (end 155.956 73.406) (width 0.4) (layer "F.Cu") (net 22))
 (segment (start 142.866 81.078) (end 142.866 79.638) (width 0.4) (layer "F.Cu") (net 22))
 (segment (start 142.866 79.638) (end 143.002 79.502) (width 0.4) (layer "F.Cu") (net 22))
 (segment (start 143.002 79.502) (end 149.86 79.502) (width 0.4) (layer "F.Cu") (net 22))
 (segment (start 134.866 73.922) (end 135.636 73.152) (width 0.4) (layer "F.Cu") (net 30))
 (segment (start 134.866 81.078) (end 134.866 73.922) (width 0.4) (layer "F.Cu") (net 30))
 (segment (start 136.866 86.816) (end 136.866 92.289) (width 0.4) (layer "F.Cu") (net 13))
 (segment (start 139.065 92.837) (end 140.716 94.488) (width 0.4) (layer "F.Cu") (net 13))
 (segment (start 137.414 92.837) (end 139.065 92.837) (width 0.4) (layer "F.Cu") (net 13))
 (segment (start 136.866 92.289) (end 137.414 92.837) (width 0.4) (layer "F.Cu") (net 13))
 (segment (start 128.4605 77.216) (end 124.206 77.216) (width 0.4) (layer "F.Cu") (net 36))
 (segment (start 124.206 77.216) (end 120.396 73.406) (width 0.4) (layer "F.Cu") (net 36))
 (segment (start 128.866 77.6215) (end 128.4605 77.216) (width 0.4) (layer "F.Cu") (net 36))
 (segment (start 128.866 81.078) (end 128.866 77.6215) (width 0.4) (layer "F.Cu") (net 36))
 (segment (start 118.162 81.078) (end 110.236 73.152) (width 0.4) (layer "F.Cu") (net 40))
 (segment (start 124.866 81.078) (end 118.162 81.078) (width 0.4) (layer "F.Cu") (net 40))
 (segment (start 128.4605 90.678) (end 124.206 90.678) (width 0.4) (layer "F.Cu") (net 5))
 (segment (start 124.206 90.678) (end 120.396 94.488) (width 0.4) (layer "F.Cu") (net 5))
 (segment (start 128.866 86.816) (end 128.866 90.2725) (width 0.4) (layer "F.Cu") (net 5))
 (segment (start 128.866 90.2725) (end 128.4605 90.678) (width 0.4) (layer "F.Cu") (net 5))
 (segment (start 118.872 88.392) (end 112.776 94.488) (width 0.4) (layer "F.Cu") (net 2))
 (segment (start 125.866 88.256) (end 125.73 88.392) (width 0.4) (layer "F.Cu") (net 2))
 (segment (start 125.73 88.392) (end 118.872 88.392) (width 0.4) (layer "F.Cu") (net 2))
 (segment (start 125.866 86.816) (end 125.866 88.256) (width 0.4) (layer "F.Cu") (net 2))
 (segment (start 138.866 76.78) (end 139.192 76.454) (width 0.4) (layer "F.Cu") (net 26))
 (segment (start 138.866 81.078) (end 138.866 76.78) (width 0.4) (layer "F.Cu") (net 26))
 (segment (start 139.192 76.454) (end 142.748 76.454) (width 0.4) (layer "F.Cu") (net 26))
 (segment (start 142.748 76.454) (end 145.796 73.406) (width 0.4) (layer "F.Cu") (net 26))
 (segment (start 137.866 76.383) (end 138.557 75.692) (width 0.4) (layer "F.Cu") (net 27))
 (segment (start 138.557 75.692) (end 140.97 75.692) (width 0.4) (layer "F.Cu") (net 27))
 (segment (start 137.866 81.078) (end 137.866 76.383) (width 0.4) (layer "F.Cu") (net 27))
 (segment (start 140.97 75.692) (end 143.256 73.406) (width 0.4) (layer "F.Cu") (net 27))
 (segment (start 120.65 89.154) (end 115.316 94.488) (width 0.4) (layer "F.Cu") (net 3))
 (segment (start 126.866 86.816) (end 126.866 88.78) (width 0.4) (layer "F.Cu") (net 3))
 (segment (start 126.866 88.78) (end 126.492 89.154) (width 0.4) (layer "F.Cu") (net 3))
 (segment (start 126.492 89.154) (end 120.65 89.154) (width 0.4) (layer "F.Cu") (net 3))
 (segment (start 142.24 89.154) (end 148.082 89.154) (width 0.4) (layer "F.Cu") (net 18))
 (segment (start 148.082 89.154) (end 153.416 94.488) (width 0.4) (layer "F.Cu") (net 18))
 (segment (start 141.866 86.816) (end 141.866 88.78) (width 0.4) (layer "F.Cu") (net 18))
 (segment (start 141.866 88.78) (end 142.24 89.154) (width 0.4) (layer "F.Cu") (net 18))
 (segment (start 120.65 78.74) (end 115.316 73.406) (width 0.4) (layer "F.Cu") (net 38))
 (segment (start 126.866 81.078) (end 126.866 79.114) (width 0.4) (layer "F.Cu") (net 38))
 (segment (start 126.866 79.114) (end 126.492 78.74) (width 0.4) (layer "F.Cu") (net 38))
 (segment (start 126.492 78.74) (end 120.65 78.74) (width 0.4) (layer "F.Cu") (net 38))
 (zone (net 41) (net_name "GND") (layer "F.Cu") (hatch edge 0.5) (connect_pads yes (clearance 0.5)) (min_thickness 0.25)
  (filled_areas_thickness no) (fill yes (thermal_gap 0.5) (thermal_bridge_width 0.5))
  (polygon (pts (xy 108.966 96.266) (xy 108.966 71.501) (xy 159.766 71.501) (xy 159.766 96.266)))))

